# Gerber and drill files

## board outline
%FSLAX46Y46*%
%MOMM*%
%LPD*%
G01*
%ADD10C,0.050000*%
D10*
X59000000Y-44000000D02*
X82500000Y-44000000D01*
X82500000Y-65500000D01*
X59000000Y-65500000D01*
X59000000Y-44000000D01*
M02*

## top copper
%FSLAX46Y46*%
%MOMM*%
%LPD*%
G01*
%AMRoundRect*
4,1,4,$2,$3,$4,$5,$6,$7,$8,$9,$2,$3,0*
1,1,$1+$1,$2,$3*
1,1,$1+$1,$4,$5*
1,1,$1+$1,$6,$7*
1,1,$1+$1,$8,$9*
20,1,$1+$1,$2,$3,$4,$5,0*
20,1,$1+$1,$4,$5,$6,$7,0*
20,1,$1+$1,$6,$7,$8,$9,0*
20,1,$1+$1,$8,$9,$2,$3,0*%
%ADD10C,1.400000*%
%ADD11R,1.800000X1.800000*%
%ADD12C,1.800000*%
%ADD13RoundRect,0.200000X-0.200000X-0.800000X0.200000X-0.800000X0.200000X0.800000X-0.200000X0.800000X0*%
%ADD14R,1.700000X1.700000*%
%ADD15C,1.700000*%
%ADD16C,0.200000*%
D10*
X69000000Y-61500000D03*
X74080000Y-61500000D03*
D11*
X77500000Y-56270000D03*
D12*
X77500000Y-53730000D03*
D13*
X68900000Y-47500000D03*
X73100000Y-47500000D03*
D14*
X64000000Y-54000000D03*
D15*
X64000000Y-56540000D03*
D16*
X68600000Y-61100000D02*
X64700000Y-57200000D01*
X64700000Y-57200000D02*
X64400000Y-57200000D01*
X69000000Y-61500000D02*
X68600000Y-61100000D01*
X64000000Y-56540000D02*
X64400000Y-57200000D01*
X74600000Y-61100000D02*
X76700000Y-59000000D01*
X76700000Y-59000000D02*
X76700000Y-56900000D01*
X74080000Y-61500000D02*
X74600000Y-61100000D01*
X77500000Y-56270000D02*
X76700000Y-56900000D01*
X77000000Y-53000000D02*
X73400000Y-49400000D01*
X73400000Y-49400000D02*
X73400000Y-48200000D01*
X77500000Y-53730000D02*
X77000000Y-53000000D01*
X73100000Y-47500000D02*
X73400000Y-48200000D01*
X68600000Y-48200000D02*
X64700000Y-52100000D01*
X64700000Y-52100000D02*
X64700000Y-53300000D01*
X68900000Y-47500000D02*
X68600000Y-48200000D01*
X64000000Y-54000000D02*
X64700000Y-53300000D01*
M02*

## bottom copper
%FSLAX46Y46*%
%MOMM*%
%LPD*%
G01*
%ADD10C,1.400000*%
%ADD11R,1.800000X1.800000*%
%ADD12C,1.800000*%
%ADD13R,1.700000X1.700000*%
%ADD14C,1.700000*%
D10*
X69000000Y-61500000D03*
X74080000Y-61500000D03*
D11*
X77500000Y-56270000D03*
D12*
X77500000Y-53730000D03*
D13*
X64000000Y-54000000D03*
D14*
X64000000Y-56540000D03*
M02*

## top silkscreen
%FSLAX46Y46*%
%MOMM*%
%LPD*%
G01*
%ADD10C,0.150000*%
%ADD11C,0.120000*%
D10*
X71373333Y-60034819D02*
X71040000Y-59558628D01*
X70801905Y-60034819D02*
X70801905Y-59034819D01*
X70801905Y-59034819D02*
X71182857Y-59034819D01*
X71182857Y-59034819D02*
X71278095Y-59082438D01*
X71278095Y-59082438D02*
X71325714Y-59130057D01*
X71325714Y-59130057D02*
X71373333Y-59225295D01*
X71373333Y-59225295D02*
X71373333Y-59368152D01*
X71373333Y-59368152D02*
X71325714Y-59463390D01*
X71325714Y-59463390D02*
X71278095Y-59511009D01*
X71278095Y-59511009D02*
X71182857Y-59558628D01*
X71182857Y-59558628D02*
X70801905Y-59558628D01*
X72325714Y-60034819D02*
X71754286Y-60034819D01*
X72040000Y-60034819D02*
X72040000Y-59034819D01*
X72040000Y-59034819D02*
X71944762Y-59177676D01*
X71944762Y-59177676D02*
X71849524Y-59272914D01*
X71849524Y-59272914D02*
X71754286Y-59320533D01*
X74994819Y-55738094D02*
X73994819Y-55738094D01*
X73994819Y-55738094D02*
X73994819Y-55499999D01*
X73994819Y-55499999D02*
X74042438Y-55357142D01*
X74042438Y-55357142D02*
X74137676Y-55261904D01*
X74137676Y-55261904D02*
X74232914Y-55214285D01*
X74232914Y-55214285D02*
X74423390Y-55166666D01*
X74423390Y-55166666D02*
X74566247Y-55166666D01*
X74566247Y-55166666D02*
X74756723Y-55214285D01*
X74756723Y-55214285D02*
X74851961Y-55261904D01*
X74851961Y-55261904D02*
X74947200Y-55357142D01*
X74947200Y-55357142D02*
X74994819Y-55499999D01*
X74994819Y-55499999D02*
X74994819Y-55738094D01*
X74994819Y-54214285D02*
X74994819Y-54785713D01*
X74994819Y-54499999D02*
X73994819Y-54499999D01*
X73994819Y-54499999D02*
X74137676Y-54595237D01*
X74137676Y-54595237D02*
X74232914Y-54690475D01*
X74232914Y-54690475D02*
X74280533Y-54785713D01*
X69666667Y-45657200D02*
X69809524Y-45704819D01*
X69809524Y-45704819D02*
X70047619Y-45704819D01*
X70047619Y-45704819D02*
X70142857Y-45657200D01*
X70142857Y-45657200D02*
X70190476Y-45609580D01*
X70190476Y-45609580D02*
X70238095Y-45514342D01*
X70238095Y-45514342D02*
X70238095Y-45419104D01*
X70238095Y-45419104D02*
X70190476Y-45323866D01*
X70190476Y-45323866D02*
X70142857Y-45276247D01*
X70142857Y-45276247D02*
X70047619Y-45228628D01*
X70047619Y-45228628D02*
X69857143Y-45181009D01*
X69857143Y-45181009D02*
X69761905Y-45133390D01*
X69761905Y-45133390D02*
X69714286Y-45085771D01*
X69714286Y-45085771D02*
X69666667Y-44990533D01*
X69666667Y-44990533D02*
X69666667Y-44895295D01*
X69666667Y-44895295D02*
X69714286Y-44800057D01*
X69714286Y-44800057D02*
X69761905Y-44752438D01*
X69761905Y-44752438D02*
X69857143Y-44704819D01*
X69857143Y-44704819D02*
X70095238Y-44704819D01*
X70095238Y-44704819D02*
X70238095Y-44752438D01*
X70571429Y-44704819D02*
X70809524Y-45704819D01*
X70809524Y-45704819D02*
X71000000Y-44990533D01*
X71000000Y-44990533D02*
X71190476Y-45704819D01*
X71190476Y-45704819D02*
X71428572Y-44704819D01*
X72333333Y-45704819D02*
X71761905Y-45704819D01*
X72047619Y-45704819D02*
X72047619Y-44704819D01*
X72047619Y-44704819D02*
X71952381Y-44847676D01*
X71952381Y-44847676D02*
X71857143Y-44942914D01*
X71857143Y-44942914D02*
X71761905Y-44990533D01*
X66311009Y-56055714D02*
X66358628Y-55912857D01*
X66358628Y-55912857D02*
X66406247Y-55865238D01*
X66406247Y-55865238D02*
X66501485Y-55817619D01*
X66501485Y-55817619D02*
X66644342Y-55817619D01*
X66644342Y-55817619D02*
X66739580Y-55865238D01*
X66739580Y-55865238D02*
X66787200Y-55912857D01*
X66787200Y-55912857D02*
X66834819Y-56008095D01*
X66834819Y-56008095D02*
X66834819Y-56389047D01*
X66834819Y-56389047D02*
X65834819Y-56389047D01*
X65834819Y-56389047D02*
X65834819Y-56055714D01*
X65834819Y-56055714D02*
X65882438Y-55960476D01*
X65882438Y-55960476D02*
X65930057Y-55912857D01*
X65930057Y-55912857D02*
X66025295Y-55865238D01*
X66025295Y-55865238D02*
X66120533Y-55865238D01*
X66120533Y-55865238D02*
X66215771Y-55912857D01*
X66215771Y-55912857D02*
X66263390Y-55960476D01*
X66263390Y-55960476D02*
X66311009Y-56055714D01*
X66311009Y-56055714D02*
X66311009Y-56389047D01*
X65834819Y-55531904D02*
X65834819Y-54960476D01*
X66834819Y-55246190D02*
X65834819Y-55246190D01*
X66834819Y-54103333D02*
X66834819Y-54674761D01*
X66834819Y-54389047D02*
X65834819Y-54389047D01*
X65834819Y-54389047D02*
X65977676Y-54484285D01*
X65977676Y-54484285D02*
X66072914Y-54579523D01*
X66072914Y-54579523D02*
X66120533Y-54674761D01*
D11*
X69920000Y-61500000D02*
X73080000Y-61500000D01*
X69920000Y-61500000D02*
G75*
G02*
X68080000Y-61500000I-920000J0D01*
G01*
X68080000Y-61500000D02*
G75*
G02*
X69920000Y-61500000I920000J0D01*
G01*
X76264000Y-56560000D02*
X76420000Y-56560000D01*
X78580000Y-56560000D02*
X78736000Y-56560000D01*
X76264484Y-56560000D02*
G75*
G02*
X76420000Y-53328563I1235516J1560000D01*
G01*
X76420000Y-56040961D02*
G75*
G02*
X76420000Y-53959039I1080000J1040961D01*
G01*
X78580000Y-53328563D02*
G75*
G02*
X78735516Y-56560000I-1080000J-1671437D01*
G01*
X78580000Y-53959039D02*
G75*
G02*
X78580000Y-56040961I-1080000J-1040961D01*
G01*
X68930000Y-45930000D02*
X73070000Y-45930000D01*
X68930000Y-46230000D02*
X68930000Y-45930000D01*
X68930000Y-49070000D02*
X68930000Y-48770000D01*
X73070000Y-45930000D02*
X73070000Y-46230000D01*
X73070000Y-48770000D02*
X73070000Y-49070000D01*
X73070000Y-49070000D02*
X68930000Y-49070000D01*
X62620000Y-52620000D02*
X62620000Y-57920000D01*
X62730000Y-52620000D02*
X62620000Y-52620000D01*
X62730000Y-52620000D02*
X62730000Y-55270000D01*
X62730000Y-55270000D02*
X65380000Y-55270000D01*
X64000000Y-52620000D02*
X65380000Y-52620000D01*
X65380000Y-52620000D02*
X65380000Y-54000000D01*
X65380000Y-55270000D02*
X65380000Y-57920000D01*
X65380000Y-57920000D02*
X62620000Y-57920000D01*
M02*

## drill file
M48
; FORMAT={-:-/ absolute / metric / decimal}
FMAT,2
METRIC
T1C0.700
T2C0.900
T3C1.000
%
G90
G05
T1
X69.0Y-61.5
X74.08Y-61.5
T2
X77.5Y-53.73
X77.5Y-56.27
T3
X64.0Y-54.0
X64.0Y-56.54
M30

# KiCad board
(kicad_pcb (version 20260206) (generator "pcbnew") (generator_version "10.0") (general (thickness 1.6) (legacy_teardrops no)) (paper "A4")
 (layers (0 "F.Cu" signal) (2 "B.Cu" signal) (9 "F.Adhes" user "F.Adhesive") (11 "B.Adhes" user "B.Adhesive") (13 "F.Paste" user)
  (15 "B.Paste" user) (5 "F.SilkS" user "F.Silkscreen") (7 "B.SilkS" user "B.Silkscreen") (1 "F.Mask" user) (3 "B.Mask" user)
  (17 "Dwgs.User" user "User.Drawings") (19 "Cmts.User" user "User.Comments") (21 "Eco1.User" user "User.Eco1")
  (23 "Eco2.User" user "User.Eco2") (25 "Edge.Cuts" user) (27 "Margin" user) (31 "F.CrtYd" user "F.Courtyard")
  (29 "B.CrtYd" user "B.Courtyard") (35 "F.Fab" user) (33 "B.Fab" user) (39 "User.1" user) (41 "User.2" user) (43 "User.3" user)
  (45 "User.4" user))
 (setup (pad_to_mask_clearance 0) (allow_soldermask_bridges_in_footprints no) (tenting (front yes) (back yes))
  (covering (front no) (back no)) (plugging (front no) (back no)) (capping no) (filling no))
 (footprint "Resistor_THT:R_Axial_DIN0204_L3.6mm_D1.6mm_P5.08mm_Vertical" (layer "F.Cu") (at 69 61.5)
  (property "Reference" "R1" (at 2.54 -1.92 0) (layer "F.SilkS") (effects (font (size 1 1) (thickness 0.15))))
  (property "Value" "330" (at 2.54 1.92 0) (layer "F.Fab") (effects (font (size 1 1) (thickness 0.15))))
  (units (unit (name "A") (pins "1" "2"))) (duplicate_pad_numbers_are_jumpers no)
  (fp_line (start 0.92 0) (end 4.08 0) (stroke (width 0.12) (type solid)) (layer "F.SilkS"))
  (fp_circle (center 0 0) (end 0.92 0) (stroke (width 0.12) (type solid)) (fill no) (layer "F.SilkS"))
  (pad "1" thru_hole circle (at 0 0) (size 1.4 1.4) (drill 0.7) (layers "*.Cu" "*.Mask") (remove_unused_layers no) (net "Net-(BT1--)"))
  (pad "2" thru_hole circle (at 5.08 0) (size 1.4 1.4) (drill 0.7) (layers "*.Cu" "*.Mask") (remove_unused_layers no) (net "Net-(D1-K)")))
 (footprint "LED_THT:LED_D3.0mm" (layer "F.Cu") (at 77.5 56.27 90)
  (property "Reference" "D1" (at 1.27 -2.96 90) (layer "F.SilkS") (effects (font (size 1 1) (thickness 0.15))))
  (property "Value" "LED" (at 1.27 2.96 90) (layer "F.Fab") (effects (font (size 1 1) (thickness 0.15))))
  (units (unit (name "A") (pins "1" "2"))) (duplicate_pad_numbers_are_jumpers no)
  (fp_line (start -0.29 -1.236) (end -0.29 -1.08) (stroke (width 0.12) (type solid)) (layer "F.SilkS"))
  (fp_line (start -0.29 1.08) (end -0.29 1.236) (stroke (width 0.12) (type solid)) (layer "F.SilkS"))
  (fp_arc (start -0.29 -1.235516) (mid 1.36566 -1.987699) (end 2.941437 -1.08) (stroke (width 0.12) (type solid)) (layer "F.SilkS"))
  (fp_arc (start 0.229039 -1.08) (mid 1.27 -1.5) (end 2.310961 -1.08) (stroke (width 0.12) (type solid)) (layer "F.SilkS"))
  (fp_arc (start 2.941437 1.08) (mid 1.36566 1.987699) (end -0.29 1.235516) (stroke (width 0.12) (type solid)) (layer "F.SilkS"))
  (fp_arc (start 2.310961 1.08) (mid 1.27 1.5) (end 0.229039 1.08) (stroke (width 0.12) (type solid)) (layer "F.SilkS"))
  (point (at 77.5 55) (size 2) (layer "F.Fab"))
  (pad "1" thru_hole rect (at 0 0 90) (size 1.8 1.8) (drill 0.9) (layers "*.Cu" "*.Mask") (remove_unused_layers no) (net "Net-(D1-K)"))
  (pad "2" thru_hole circle (at 2.54 0 90) (size 1.8 1.8) (drill 0.9) (layers "*.Cu" "*.Mask") (remove_unused_layers no) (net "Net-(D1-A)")))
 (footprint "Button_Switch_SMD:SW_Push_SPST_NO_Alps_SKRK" (layer "F.Cu") (at 71 47.5)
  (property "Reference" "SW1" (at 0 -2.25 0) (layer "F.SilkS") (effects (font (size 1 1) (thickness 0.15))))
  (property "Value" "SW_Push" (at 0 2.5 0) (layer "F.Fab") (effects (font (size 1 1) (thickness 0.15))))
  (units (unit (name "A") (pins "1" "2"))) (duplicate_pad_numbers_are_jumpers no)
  (fp_line (start -2.07 -1.57) (end 2.07 -1.57) (stroke (width 0.12) (type solid)) (layer "F.SilkS"))
  (fp_line (start -2.07 -1.27) (end -2.07 -1.57) (stroke (width 0.12) (type solid)) (layer "F.SilkS"))
  (fp_line (start -2.07 1.57) (end -2.07 1.27) (stroke (width 0.12) (type solid)) (layer "F.SilkS"))
  (fp_line (start 2.07 -1.57) (end 2.07 -1.27) (stroke (width 0.12) (type solid)) (layer "F.SilkS"))
  (fp_line (start 2.07 1.27) (end 2.07 1.57) (stroke (width 0.12) (type solid)) (layer "F.SilkS"))
  (fp_line (start 2.07 1.57) (end -2.07 1.57) (stroke (width 0.12) (type solid)) (layer "F.SilkS"))
  (pad "1" smd roundrect (at -2.1 0) (size 0.8 2) (layers "F.Cu" "F.Mask" "F.Paste") (roundrect_rratio 0.25) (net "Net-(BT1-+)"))
  (pad "2" smd roundrect (at 2.1 0) (size 0.8 2) (layers "F.Cu" "F.Mask" "F.Paste") (roundrect_rratio 0.25) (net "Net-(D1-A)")))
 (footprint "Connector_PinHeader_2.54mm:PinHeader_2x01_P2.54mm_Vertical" (layer "F.Cu") (at 64 54 -90)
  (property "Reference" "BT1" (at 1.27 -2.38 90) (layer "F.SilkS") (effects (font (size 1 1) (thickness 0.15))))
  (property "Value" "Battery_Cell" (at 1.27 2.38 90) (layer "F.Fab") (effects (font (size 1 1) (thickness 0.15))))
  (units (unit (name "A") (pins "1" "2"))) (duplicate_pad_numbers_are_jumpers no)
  (fp_line (start -1.38 1.38) (end 3.92 1.38) (stroke (width 0.12) (type solid)) (layer "F.SilkS"))
  (fp_line (start -1.38 1.27) (end -1.38 1.38) (stroke (width 0.12) (type solid)) (layer "F.SilkS"))
  (fp_line (start -1.38 1.27) (end 1.27 1.27) (stroke (width 0.12) (type solid)) (layer "F.SilkS"))
  (fp_line (start 1.27 1.27) (end 1.27 -1.38) (stroke (width 0.12) (type solid)) (layer "F.SilkS"))
  (fp_line (start -1.38 0) (end -1.38 -1.38) (stroke (width 0.12) (type solid)) (layer "F.SilkS"))
  (fp_line (start -1.38 -1.38) (end 0 -1.38) (stroke (width 0.12) (type solid)) (layer "F.SilkS"))
  (fp_line (start 1.27 -1.38) (end 3.92 -1.38) (stroke (width 0.12) (type solid)) (layer "F.SilkS"))
  (fp_line (start 3.92 -1.38) (end 3.92 1.38) (stroke (width 0.12) (type solid)) (layer "F.SilkS"))
  (pad "1" thru_hole rect (at 0 0 270) (size 1.7 1.7) (drill 1) (layers "*.Cu" "*.Mask") (remove_unused_layers no) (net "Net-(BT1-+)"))
  (pad "2" thru_hole circle (at 2.54 0 270) (size 1.7 1.7) (drill 1) (layers "*.Cu" "*.Mask") (remove_unused_layers no) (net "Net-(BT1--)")))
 (gr_rect (start 59 44) (end 82.5 65.5) (stroke (width 0.05) (type default)) (fill no) (layer "Edge.Cuts"))
 (segment (start 68.6 61.099999999999994) (end 64.7 57.2) (width 0.2) (layer "F.Cu") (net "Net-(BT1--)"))
 (segment (start 64.7 57.2) (end 64.4 57.2) (width 0.2) (layer "F.Cu") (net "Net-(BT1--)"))
 (segment (start 69 61.5) (end 68.6 61.099999999999994) (width 0.2) (layer "F.Cu") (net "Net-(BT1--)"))
 (segment (start 64 56.54) (end 64.4 57.2) (width 0.2) (layer "F.Cu") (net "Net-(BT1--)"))
 (segment (start 74.6 61.099999999999994) (end 76.7 59) (width 0.2) (layer "F.Cu") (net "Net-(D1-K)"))
 (segment (start 76.7 59) (end 76.7 56.9) (width 0.2) (layer "F.Cu") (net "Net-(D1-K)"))
 (segment (start 74.08 61.5) (end 74.6 61.099999999999994) (width 0.2) (layer "F.Cu") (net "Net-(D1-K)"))
 (segment (start 77.5 56.27) (end 76.7 56.9) (width 0.2) (layer "F.Cu") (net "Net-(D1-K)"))
 (segment (start 77 53) (end 73.4 49.4) (width 0.2) (layer "F.Cu") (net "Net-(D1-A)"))
 (segment (start 73.4 49.4) (end 73.4 48.2) (width 0.2) (layer "F.Cu") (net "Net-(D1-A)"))
 (segment (start 77.5 53.730000000000004) (end 77 53) (width 0.2) (layer "F.Cu") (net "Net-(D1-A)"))
 (segment (start 73.1 47.5) (end 73.4 48.2) (width 0.2) (layer "F.Cu") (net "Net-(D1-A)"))
 (segment (start 68.6 48.2) (end 64.7 52.1) (width 0.2) (layer "F.Cu") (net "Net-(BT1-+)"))
 (segment (start 64.7 52.1) (end 64.7 53.3) (width 0.2) (layer "F.Cu") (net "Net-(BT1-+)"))
 (segment (start 68.9 47.5) (end 68.6 48.2) (width 0.2) (layer "F.Cu") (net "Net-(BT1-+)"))
 (segment (start 64 54) (end 64.7 53.3) (width 0.2) (layer "F.Cu") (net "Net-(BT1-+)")))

